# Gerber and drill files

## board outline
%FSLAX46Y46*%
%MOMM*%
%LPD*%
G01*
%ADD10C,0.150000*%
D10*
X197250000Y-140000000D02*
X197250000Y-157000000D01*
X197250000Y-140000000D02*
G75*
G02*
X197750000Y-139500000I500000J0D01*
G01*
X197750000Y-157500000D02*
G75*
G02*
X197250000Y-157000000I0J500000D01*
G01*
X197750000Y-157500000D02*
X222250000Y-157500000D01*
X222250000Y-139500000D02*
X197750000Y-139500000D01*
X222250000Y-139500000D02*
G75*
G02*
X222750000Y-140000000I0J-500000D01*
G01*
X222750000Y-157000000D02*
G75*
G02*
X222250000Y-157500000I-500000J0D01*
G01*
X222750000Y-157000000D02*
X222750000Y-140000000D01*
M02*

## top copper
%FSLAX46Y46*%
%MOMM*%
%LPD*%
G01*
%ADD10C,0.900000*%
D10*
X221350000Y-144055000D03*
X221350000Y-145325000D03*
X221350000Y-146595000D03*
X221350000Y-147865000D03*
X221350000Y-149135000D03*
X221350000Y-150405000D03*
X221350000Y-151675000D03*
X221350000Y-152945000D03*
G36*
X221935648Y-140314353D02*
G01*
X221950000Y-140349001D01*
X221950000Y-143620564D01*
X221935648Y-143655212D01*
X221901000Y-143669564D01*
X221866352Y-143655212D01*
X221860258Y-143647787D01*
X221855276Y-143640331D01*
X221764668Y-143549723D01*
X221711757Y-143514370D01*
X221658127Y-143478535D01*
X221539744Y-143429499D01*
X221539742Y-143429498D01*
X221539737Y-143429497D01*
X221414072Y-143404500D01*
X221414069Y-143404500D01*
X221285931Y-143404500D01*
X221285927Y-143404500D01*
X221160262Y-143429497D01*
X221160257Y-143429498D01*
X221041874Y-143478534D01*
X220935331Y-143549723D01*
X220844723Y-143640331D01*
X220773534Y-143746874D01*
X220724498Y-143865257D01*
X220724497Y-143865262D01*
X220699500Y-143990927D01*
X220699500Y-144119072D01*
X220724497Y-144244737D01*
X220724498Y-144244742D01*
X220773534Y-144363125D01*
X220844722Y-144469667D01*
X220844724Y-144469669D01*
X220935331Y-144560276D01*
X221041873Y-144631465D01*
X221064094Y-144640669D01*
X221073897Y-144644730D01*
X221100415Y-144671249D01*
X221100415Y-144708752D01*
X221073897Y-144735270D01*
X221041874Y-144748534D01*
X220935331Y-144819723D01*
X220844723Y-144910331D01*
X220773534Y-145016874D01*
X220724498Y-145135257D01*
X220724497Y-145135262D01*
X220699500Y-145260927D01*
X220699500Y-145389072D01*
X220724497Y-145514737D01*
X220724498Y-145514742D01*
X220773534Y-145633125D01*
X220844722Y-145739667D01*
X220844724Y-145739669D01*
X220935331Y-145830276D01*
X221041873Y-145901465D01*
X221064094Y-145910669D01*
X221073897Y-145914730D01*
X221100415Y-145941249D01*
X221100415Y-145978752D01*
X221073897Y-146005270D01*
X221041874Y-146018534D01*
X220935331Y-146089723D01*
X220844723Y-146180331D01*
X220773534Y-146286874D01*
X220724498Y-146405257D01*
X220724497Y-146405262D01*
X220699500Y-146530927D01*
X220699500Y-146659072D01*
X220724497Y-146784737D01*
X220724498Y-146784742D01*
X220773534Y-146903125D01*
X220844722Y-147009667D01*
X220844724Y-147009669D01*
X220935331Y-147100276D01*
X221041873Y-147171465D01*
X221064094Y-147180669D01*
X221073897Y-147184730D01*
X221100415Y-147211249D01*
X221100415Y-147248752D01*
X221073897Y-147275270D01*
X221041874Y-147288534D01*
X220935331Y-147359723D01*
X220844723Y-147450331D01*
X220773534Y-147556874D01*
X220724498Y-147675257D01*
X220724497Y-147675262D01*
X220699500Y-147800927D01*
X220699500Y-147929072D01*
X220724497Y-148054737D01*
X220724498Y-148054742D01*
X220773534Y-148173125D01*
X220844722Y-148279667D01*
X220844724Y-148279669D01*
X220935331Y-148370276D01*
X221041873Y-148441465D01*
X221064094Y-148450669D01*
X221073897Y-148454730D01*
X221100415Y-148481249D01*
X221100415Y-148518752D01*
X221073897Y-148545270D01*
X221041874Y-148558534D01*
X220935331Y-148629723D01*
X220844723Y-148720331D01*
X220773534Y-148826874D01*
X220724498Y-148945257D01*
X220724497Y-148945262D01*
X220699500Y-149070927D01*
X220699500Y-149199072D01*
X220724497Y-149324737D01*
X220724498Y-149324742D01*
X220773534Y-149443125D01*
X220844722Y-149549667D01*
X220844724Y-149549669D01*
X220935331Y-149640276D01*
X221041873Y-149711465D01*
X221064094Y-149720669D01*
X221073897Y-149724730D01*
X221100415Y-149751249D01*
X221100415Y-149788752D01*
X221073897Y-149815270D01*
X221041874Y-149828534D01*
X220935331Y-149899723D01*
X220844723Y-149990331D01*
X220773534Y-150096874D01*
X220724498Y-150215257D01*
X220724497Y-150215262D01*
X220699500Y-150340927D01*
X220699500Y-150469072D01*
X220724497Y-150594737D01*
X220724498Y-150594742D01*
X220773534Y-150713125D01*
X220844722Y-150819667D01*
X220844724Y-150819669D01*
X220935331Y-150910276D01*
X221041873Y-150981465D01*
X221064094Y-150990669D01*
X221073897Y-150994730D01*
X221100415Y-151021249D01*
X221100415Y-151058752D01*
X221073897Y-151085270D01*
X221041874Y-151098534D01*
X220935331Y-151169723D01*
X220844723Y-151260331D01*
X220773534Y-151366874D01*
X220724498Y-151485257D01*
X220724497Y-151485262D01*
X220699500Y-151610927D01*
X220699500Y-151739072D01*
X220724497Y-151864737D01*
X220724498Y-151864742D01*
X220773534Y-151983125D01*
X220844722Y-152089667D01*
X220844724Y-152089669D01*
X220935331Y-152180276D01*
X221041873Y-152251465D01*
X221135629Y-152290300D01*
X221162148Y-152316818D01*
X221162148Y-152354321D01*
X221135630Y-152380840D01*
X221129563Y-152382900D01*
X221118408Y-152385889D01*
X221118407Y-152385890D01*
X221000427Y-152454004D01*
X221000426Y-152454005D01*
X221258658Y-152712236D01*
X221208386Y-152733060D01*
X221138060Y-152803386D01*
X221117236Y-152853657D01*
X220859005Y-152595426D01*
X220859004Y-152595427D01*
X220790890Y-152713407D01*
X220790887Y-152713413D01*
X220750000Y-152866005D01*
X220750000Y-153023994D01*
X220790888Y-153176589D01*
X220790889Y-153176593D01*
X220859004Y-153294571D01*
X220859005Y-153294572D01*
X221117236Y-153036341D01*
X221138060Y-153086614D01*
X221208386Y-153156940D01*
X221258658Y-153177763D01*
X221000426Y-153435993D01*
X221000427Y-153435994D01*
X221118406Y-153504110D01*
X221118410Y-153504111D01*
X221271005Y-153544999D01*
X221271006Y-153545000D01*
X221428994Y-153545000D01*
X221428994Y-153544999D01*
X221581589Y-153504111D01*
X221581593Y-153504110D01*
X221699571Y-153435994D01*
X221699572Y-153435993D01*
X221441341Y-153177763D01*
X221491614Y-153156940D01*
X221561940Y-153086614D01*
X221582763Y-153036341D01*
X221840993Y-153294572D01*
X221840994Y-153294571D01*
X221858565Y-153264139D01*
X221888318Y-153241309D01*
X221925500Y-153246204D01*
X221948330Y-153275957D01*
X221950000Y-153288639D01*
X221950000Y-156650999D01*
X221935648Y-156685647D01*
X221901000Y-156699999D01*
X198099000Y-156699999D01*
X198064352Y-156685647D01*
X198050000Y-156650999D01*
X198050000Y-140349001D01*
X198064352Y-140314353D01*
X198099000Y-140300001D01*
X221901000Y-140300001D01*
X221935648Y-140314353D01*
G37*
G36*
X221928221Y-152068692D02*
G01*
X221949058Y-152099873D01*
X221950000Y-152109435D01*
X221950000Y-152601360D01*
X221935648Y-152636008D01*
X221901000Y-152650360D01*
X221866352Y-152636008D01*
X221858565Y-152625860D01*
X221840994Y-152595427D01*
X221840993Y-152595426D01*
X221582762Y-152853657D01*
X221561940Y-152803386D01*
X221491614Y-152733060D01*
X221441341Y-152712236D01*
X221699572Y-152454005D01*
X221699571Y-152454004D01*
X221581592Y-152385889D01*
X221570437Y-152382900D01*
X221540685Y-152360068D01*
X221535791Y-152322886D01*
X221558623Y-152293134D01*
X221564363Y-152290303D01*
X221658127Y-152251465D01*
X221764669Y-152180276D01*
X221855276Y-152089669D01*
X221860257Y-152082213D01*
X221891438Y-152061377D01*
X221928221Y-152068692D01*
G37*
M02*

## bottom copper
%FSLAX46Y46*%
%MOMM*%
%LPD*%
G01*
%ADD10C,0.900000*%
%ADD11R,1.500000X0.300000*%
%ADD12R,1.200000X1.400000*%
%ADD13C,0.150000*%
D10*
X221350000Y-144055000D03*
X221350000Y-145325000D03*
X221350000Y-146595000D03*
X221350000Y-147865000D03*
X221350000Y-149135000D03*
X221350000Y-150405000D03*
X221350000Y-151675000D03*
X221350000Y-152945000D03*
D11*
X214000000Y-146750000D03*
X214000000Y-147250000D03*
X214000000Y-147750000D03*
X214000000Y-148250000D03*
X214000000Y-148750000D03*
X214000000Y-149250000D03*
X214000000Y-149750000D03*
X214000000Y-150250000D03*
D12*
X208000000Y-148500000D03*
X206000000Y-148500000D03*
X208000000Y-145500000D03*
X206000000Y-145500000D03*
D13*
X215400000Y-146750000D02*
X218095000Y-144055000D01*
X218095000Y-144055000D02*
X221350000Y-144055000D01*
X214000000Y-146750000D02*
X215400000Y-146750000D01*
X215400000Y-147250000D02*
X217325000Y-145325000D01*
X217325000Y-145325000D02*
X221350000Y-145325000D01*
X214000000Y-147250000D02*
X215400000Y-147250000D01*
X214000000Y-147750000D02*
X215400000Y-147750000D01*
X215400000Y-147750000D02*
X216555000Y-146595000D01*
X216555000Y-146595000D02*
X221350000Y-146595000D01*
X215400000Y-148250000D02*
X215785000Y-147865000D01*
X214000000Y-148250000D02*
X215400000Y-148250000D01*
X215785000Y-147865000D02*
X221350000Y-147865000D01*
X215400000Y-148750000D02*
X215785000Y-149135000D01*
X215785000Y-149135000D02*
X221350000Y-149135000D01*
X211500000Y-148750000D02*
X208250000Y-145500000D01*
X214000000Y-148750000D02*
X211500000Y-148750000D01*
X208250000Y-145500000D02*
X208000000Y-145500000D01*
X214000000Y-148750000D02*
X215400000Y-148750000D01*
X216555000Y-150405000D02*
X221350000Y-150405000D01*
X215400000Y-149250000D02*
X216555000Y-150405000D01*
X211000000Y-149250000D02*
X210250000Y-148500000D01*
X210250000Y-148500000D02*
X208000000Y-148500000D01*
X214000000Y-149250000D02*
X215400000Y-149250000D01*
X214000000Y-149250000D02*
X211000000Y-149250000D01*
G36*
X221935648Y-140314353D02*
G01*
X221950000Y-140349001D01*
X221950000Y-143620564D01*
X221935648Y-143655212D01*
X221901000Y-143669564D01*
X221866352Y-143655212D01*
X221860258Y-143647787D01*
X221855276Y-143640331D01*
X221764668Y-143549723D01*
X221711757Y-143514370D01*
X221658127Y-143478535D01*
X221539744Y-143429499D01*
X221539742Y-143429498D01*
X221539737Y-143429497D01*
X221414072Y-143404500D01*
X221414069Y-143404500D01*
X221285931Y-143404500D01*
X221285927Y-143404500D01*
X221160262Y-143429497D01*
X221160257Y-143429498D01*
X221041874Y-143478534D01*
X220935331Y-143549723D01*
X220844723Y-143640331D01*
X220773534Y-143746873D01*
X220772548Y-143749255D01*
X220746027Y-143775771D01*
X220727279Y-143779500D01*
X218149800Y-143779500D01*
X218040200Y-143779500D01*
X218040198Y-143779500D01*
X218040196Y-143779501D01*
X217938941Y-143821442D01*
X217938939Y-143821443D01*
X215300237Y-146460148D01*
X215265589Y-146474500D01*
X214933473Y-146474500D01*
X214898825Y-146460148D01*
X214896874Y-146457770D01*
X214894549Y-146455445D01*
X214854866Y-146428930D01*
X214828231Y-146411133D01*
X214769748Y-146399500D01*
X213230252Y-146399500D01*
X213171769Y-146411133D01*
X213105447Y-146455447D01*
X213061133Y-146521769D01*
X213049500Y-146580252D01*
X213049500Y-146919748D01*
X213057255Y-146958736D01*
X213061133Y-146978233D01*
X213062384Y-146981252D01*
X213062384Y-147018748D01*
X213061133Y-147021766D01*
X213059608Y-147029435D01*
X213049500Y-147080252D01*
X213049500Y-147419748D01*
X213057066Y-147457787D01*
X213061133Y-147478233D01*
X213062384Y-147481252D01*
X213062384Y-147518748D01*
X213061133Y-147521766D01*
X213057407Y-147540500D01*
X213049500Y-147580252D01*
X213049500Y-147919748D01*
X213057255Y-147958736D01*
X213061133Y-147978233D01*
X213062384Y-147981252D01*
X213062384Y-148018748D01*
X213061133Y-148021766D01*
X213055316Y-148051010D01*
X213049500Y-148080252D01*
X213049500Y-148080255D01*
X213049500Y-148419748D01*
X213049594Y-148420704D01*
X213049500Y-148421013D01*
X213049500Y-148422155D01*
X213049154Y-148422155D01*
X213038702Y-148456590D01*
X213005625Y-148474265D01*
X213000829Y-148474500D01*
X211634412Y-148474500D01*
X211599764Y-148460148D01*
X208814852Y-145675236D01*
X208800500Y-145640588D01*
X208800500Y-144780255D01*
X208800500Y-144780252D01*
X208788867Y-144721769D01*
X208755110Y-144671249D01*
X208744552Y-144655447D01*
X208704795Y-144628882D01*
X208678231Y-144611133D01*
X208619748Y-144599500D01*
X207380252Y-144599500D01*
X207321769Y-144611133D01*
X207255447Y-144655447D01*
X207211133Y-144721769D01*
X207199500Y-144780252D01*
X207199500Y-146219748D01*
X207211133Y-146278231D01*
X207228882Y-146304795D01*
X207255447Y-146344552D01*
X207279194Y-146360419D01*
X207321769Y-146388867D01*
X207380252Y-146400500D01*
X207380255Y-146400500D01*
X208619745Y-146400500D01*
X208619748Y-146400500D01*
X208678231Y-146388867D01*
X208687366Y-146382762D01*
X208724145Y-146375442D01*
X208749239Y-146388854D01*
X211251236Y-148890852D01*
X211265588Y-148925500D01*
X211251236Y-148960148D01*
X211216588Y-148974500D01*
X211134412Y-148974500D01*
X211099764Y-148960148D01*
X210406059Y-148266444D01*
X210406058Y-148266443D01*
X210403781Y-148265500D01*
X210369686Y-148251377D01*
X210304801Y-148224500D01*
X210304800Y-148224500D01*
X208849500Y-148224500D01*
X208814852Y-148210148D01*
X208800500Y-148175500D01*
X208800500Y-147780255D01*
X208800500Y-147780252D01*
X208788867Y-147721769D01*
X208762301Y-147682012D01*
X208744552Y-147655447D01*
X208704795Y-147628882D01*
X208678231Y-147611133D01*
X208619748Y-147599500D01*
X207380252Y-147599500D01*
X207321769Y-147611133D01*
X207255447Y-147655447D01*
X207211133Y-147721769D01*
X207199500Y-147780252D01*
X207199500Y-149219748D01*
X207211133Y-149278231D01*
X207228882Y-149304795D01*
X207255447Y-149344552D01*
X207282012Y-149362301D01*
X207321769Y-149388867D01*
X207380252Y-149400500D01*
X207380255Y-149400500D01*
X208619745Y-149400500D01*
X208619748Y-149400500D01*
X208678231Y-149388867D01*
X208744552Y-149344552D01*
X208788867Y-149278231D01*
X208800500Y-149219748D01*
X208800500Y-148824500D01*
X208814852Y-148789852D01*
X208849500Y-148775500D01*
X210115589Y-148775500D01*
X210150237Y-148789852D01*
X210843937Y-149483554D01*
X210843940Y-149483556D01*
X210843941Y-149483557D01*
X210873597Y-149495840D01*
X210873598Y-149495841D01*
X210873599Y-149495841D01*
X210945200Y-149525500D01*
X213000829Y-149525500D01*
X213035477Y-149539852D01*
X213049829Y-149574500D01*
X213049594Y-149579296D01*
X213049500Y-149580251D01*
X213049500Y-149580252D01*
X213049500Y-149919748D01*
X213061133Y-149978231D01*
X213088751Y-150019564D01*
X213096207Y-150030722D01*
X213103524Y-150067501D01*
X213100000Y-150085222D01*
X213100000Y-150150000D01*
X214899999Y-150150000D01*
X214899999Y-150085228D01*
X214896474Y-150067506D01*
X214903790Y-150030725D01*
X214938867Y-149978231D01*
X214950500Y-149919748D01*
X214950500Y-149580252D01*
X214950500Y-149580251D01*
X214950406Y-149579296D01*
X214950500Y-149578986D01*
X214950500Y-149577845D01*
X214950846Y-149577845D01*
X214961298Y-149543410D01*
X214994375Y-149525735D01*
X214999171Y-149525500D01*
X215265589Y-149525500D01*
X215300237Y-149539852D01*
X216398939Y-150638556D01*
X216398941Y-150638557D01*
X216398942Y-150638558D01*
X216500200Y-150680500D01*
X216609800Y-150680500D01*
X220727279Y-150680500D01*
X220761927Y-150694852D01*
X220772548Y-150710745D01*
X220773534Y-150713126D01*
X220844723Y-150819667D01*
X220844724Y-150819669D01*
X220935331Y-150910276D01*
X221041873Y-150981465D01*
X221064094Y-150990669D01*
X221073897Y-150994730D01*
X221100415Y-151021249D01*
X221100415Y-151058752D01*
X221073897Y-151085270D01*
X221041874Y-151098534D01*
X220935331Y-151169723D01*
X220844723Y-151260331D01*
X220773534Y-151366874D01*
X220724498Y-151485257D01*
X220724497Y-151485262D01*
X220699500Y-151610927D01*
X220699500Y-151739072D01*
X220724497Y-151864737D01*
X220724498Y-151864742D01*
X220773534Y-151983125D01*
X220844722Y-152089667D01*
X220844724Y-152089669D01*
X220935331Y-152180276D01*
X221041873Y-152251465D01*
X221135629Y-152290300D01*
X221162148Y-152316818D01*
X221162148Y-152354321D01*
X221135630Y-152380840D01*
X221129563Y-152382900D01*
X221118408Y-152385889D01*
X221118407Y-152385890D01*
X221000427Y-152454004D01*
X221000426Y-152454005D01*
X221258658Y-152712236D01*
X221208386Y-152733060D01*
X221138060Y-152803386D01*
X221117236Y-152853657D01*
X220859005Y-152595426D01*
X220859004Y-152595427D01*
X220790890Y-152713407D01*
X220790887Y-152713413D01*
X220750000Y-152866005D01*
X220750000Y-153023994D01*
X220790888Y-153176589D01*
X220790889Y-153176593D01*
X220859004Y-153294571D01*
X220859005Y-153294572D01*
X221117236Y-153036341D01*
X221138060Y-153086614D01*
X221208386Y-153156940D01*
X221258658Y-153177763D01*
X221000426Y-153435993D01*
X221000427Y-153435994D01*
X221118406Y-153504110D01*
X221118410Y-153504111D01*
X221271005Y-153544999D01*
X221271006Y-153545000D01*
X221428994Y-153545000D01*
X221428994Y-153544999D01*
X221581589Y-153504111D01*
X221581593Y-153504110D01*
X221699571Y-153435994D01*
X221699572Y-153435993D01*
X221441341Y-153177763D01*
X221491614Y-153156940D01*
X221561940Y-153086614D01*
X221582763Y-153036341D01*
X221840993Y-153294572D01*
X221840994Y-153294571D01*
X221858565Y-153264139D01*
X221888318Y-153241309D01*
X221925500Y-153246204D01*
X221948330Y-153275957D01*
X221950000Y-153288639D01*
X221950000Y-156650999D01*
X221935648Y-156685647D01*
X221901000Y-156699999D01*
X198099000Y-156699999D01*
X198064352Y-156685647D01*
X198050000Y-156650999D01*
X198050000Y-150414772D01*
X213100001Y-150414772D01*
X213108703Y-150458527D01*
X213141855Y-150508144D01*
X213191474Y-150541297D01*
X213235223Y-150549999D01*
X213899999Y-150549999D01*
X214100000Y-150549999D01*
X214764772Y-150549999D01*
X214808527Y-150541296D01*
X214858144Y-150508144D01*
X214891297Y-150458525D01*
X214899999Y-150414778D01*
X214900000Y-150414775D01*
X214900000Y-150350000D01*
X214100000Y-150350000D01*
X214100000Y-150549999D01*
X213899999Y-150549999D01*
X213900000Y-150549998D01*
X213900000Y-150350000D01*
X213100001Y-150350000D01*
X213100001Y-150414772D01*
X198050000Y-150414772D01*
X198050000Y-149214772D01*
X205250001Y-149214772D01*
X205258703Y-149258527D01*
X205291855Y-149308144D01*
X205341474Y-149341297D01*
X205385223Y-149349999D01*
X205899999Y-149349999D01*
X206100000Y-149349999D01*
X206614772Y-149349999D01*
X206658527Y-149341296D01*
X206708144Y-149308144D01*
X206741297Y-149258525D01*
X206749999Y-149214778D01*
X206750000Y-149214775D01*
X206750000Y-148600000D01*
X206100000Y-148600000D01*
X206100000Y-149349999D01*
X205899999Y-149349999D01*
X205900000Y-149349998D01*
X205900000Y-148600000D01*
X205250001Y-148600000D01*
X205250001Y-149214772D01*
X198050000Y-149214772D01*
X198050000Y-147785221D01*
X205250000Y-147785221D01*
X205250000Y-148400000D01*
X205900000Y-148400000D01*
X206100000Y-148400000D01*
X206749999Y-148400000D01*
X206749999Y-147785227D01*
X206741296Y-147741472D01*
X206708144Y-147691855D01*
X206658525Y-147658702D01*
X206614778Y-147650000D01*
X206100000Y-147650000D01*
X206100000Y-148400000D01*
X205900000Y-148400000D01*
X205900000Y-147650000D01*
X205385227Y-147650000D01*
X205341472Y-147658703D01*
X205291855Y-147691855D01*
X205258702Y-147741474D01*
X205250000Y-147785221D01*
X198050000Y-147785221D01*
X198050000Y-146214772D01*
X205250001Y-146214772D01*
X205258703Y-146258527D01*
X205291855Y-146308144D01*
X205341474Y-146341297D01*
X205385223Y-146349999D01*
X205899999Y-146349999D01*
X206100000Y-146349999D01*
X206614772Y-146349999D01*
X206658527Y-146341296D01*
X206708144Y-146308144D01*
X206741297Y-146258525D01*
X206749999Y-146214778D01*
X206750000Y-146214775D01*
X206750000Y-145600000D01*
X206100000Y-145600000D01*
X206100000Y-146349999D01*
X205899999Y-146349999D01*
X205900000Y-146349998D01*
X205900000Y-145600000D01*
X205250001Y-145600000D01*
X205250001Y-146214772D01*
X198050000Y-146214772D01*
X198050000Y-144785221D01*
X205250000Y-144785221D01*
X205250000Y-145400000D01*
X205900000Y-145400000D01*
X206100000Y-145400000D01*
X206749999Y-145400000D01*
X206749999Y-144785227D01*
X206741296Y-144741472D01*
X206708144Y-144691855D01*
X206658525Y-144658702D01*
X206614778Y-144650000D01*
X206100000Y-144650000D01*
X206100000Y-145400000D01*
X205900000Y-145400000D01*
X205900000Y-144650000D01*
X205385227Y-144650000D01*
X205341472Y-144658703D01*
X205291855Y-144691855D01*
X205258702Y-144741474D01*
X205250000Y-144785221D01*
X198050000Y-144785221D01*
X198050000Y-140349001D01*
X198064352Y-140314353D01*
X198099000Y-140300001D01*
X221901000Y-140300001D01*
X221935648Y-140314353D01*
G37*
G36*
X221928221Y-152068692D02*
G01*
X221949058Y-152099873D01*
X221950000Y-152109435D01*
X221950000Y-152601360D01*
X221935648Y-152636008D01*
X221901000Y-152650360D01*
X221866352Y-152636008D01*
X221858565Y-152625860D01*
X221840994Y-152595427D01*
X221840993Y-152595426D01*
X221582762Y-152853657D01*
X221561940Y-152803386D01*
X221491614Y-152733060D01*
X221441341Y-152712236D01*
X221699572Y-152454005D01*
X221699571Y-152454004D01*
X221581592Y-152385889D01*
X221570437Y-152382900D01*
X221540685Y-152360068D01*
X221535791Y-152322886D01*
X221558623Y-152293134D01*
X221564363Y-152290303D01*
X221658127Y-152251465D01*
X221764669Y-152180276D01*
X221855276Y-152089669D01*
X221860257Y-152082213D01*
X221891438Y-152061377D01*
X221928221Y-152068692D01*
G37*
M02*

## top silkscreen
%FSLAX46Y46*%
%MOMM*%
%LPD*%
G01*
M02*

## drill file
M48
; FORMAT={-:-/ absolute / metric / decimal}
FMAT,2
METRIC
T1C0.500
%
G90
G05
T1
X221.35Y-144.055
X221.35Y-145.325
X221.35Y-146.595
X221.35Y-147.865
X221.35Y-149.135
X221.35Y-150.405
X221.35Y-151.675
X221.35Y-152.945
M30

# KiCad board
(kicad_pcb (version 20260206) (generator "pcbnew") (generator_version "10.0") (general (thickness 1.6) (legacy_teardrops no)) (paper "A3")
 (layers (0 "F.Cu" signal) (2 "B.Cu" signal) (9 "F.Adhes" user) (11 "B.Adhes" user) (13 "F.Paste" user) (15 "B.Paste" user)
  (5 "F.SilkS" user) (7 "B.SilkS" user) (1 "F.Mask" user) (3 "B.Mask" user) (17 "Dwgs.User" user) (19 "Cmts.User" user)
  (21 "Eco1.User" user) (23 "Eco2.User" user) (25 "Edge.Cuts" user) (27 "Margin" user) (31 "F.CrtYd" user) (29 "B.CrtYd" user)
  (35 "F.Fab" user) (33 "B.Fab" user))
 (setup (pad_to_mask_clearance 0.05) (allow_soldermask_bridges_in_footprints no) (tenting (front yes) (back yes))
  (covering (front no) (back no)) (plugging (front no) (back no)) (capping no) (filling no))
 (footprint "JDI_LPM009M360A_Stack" (layer "F.Cu") (at 210 148.5)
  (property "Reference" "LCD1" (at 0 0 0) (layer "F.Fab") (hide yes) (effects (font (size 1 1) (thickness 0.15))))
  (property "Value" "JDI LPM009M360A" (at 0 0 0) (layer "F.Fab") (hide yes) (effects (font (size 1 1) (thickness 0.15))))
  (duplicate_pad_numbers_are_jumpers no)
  (pad "1" thru_hole circle (at 11.35 -4.445) (size 0.9 0.9) (drill 0.5) (layers "*.Cu" "*.Mask") (remove_unused_layers no) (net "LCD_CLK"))
  (pad "2" thru_hole circle (at 11.35 -3.175) (size 0.9 0.9) (drill 0.5) (layers "*.Cu" "*.Mask") (remove_unused_layers no) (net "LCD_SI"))
  (pad "3" thru_hole circle (at 11.35 -1.905) (size 0.9 0.9) (drill 0.5) (layers "*.Cu" "*.Mask") (remove_unused_layers no) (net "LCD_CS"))
  (pad "4" thru_hole circle (at 11.35 -0.635) (size 0.9 0.9) (drill 0.5) (layers "*.Cu" "*.Mask") (remove_unused_layers no) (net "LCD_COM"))
  (pad "5" thru_hole circle (at 11.35 0.635) (size 0.9 0.9) (drill 0.5) (layers "*.Cu" "*.Mask") (remove_unused_layers no) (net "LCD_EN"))
  (pad "6" thru_hole circle (at 11.35 1.905) (size 0.9 0.9) (drill 0.5) (layers "*.Cu" "*.Mask") (remove_unused_layers no) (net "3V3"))
  (pad "7" thru_hole circle (at 11.35 3.175) (size 0.9 0.9) (drill 0.5) (layers "*.Cu" "*.Mask") (remove_unused_layers no))
  (pad "8" thru_hole circle (at 11.35 4.445) (size 0.9 0.9) (drill 0.5) (layers "*.Cu" "*.Mask") (remove_unused_layers no) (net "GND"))
  (pad "9" smd rect (at 4 -1.75) (size 1.5 0.3) (layers "B.Cu" "B.Mask" "B.Paste") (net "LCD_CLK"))
  (pad "10" smd rect (at 4 -1.25) (size 1.5 0.3) (layers "B.Cu" "B.Mask" "B.Paste") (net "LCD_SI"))
  (pad "11" smd rect (at 4 -0.75) (size 1.5 0.3) (layers "B.Cu" "B.Mask" "B.Paste") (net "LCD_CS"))
  (pad "12" smd rect (at 4 -0.25) (size 1.5 0.3) (layers "B.Cu" "B.Mask" "B.Paste") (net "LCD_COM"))
  (pad "13" smd rect (at 4 0.25) (size 1.5 0.3) (layers "B.Cu" "B.Mask" "B.Paste") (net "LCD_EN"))
  (pad "14" smd rect (at 4 0.75) (size 1.5 0.3) (layers "B.Cu" "B.Mask" "B.Paste") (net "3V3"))
  (pad "15" smd rect (at 4 1.25) (size 1.5 0.3) (layers "B.Cu" "B.Mask" "B.Paste"))
  (pad "16" smd rect (at 4 1.75) (size 1.5 0.3) (layers "B.Cu" "B.Mask" "B.Paste") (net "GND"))
  (pad "17" smd rect (at -2 0) (size 1.2 1.4) (layers "B.Cu" "B.Mask" "B.Paste") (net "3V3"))
  (pad "18" smd rect (at -4 0) (size 1.2 1.4) (layers "B.Cu" "B.Mask" "B.Paste") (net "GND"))
  (pad "19" smd rect (at -2 -3) (size 1.2 1.4) (layers "B.Cu" "B.Mask" "B.Paste") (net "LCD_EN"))
  (pad "20" smd rect (at -4 -3) (size 1.2 1.4) (layers "B.Cu" "B.Mask" "B.Paste") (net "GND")))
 (gr_line (start 197.25 140) (end 197.25 157) (stroke (width 0.15) (type solid)) (layer "Edge.Cuts"))
 (gr_arc (start 197.25 140) (mid 197.396447 139.646447) (end 197.75 139.5) (stroke (width 0.15) (type solid)) (layer "Edge.Cuts"))
 (gr_arc (start 197.75 157.5) (mid 197.396447 157.353553) (end 197.25 157) (stroke (width 0.15) (type solid)) (layer "Edge.Cuts"))
 (gr_line (start 197.75 157.5) (end 222.25 157.5) (stroke (width 0.15) (type solid)) (layer "Edge.Cuts"))
 (gr_line (start 222.25 139.5) (end 197.75 139.5) (stroke (width 0.15) (type solid)) (layer "Edge.Cuts"))
 (gr_arc (start 222.25 139.5) (mid 222.603553 139.646447) (end 222.75 140) (stroke (width 0.15) (type solid)) (layer "Edge.Cuts"))
 (gr_arc (start 222.75 157) (mid 222.603553 157.353553) (end 222.25 157.5) (stroke (width 0.15) (type solid)) (layer "Edge.Cuts"))
 (gr_line (start 222.75 157) (end 222.75 140) (stroke (width 0.15) (type solid)) (layer "Edge.Cuts"))
 (segment (start 215.4 146.75) (end 218.095 144.055) (width 0.15) (layer "B.Cu") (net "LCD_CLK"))
 (segment (start 218.095 144.055) (end 221.35 144.055) (width 0.15) (layer "B.Cu") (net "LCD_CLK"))
 (segment (start 214 146.75) (end 215.4 146.75) (width 0.15) (layer "B.Cu") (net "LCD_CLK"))
 (segment (start 215.4 147.25) (end 217.325 145.325) (width 0.15) (layer "B.Cu") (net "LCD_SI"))
 (segment (start 217.325 145.325) (end 221.35 145.325) (width 0.15) (layer "B.Cu") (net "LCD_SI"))
 (segment (start 214 147.25) (end 215.4 147.25) (width 0.15) (layer "B.Cu") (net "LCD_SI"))
 (segment (start 214 147.75) (end 215.4 147.75) (width 0.15) (layer "B.Cu") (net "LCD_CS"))
 (segment (start 215.4 147.75) (end 216.555 146.595) (width 0.15) (layer "B.Cu") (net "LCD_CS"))
 (segment (start 216.555 146.595) (end 221.35 146.595) (width 0.15) (layer "B.Cu") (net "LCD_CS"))
 (segment (start 215.4 148.25) (end 215.785 147.865) (width 0.15) (layer "B.Cu") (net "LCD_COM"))
 (segment (start 214 148.25) (end 215.4 148.25) (width 0.15) (layer "B.Cu") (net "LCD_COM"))
 (segment (start 215.785 147.865) (end 221.35 147.865) (width 0.15) (layer "B.Cu") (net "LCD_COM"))
 (segment (start 215.4 148.75) (end 215.785 149.135) (width 0.15) (layer "B.Cu") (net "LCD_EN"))
 (segment (start 215.785 149.135) (end 221.35 149.135) (width 0.15) (layer "B.Cu") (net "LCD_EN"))
 (segment (start 211.5 148.75) (end 208.25 145.5) (width 0.15) (layer "B.Cu") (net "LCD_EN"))
 (segment (start 214 148.75) (end 211.5 148.75) (width 0.15) (layer "B.Cu") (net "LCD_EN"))
 (segment (start 208.25 145.5) (end 208 145.5) (width 0.15) (layer "B.Cu") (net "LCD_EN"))
 (segment (start 214 148.75) (end 215.4 148.75) (width 0.15) (layer "B.Cu") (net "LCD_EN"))
 (segment (start 216.555 150.405) (end 221.35 150.405) (width 0.15) (layer "B.Cu") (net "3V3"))
 (segment (start 215.4 149.25) (end 216.555 150.405) (width 0.15) (layer "B.Cu") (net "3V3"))
 (segment (start 211 149.25) (end 210.25 148.5) (width 0.15) (layer "B.Cu") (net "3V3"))
 (segment (start 210.25 148.5) (end 208 148.5) (width 0.15) (layer "B.Cu") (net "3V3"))
 (segment (start 214 149.25) (end 215.4 149.25) (width 0.15) (layer "B.Cu") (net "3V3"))
 (segment (start 214 149.25) (end 211 149.25) (width 0.15) (layer "B.Cu") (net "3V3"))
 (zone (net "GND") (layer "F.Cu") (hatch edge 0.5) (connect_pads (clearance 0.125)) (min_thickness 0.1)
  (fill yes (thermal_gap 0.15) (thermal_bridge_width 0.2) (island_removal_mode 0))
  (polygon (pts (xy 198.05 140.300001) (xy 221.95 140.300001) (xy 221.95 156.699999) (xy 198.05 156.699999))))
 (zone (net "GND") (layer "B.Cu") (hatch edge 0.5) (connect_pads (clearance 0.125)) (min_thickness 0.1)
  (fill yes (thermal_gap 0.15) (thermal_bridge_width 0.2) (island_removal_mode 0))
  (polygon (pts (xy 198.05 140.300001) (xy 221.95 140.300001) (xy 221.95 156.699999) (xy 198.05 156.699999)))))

